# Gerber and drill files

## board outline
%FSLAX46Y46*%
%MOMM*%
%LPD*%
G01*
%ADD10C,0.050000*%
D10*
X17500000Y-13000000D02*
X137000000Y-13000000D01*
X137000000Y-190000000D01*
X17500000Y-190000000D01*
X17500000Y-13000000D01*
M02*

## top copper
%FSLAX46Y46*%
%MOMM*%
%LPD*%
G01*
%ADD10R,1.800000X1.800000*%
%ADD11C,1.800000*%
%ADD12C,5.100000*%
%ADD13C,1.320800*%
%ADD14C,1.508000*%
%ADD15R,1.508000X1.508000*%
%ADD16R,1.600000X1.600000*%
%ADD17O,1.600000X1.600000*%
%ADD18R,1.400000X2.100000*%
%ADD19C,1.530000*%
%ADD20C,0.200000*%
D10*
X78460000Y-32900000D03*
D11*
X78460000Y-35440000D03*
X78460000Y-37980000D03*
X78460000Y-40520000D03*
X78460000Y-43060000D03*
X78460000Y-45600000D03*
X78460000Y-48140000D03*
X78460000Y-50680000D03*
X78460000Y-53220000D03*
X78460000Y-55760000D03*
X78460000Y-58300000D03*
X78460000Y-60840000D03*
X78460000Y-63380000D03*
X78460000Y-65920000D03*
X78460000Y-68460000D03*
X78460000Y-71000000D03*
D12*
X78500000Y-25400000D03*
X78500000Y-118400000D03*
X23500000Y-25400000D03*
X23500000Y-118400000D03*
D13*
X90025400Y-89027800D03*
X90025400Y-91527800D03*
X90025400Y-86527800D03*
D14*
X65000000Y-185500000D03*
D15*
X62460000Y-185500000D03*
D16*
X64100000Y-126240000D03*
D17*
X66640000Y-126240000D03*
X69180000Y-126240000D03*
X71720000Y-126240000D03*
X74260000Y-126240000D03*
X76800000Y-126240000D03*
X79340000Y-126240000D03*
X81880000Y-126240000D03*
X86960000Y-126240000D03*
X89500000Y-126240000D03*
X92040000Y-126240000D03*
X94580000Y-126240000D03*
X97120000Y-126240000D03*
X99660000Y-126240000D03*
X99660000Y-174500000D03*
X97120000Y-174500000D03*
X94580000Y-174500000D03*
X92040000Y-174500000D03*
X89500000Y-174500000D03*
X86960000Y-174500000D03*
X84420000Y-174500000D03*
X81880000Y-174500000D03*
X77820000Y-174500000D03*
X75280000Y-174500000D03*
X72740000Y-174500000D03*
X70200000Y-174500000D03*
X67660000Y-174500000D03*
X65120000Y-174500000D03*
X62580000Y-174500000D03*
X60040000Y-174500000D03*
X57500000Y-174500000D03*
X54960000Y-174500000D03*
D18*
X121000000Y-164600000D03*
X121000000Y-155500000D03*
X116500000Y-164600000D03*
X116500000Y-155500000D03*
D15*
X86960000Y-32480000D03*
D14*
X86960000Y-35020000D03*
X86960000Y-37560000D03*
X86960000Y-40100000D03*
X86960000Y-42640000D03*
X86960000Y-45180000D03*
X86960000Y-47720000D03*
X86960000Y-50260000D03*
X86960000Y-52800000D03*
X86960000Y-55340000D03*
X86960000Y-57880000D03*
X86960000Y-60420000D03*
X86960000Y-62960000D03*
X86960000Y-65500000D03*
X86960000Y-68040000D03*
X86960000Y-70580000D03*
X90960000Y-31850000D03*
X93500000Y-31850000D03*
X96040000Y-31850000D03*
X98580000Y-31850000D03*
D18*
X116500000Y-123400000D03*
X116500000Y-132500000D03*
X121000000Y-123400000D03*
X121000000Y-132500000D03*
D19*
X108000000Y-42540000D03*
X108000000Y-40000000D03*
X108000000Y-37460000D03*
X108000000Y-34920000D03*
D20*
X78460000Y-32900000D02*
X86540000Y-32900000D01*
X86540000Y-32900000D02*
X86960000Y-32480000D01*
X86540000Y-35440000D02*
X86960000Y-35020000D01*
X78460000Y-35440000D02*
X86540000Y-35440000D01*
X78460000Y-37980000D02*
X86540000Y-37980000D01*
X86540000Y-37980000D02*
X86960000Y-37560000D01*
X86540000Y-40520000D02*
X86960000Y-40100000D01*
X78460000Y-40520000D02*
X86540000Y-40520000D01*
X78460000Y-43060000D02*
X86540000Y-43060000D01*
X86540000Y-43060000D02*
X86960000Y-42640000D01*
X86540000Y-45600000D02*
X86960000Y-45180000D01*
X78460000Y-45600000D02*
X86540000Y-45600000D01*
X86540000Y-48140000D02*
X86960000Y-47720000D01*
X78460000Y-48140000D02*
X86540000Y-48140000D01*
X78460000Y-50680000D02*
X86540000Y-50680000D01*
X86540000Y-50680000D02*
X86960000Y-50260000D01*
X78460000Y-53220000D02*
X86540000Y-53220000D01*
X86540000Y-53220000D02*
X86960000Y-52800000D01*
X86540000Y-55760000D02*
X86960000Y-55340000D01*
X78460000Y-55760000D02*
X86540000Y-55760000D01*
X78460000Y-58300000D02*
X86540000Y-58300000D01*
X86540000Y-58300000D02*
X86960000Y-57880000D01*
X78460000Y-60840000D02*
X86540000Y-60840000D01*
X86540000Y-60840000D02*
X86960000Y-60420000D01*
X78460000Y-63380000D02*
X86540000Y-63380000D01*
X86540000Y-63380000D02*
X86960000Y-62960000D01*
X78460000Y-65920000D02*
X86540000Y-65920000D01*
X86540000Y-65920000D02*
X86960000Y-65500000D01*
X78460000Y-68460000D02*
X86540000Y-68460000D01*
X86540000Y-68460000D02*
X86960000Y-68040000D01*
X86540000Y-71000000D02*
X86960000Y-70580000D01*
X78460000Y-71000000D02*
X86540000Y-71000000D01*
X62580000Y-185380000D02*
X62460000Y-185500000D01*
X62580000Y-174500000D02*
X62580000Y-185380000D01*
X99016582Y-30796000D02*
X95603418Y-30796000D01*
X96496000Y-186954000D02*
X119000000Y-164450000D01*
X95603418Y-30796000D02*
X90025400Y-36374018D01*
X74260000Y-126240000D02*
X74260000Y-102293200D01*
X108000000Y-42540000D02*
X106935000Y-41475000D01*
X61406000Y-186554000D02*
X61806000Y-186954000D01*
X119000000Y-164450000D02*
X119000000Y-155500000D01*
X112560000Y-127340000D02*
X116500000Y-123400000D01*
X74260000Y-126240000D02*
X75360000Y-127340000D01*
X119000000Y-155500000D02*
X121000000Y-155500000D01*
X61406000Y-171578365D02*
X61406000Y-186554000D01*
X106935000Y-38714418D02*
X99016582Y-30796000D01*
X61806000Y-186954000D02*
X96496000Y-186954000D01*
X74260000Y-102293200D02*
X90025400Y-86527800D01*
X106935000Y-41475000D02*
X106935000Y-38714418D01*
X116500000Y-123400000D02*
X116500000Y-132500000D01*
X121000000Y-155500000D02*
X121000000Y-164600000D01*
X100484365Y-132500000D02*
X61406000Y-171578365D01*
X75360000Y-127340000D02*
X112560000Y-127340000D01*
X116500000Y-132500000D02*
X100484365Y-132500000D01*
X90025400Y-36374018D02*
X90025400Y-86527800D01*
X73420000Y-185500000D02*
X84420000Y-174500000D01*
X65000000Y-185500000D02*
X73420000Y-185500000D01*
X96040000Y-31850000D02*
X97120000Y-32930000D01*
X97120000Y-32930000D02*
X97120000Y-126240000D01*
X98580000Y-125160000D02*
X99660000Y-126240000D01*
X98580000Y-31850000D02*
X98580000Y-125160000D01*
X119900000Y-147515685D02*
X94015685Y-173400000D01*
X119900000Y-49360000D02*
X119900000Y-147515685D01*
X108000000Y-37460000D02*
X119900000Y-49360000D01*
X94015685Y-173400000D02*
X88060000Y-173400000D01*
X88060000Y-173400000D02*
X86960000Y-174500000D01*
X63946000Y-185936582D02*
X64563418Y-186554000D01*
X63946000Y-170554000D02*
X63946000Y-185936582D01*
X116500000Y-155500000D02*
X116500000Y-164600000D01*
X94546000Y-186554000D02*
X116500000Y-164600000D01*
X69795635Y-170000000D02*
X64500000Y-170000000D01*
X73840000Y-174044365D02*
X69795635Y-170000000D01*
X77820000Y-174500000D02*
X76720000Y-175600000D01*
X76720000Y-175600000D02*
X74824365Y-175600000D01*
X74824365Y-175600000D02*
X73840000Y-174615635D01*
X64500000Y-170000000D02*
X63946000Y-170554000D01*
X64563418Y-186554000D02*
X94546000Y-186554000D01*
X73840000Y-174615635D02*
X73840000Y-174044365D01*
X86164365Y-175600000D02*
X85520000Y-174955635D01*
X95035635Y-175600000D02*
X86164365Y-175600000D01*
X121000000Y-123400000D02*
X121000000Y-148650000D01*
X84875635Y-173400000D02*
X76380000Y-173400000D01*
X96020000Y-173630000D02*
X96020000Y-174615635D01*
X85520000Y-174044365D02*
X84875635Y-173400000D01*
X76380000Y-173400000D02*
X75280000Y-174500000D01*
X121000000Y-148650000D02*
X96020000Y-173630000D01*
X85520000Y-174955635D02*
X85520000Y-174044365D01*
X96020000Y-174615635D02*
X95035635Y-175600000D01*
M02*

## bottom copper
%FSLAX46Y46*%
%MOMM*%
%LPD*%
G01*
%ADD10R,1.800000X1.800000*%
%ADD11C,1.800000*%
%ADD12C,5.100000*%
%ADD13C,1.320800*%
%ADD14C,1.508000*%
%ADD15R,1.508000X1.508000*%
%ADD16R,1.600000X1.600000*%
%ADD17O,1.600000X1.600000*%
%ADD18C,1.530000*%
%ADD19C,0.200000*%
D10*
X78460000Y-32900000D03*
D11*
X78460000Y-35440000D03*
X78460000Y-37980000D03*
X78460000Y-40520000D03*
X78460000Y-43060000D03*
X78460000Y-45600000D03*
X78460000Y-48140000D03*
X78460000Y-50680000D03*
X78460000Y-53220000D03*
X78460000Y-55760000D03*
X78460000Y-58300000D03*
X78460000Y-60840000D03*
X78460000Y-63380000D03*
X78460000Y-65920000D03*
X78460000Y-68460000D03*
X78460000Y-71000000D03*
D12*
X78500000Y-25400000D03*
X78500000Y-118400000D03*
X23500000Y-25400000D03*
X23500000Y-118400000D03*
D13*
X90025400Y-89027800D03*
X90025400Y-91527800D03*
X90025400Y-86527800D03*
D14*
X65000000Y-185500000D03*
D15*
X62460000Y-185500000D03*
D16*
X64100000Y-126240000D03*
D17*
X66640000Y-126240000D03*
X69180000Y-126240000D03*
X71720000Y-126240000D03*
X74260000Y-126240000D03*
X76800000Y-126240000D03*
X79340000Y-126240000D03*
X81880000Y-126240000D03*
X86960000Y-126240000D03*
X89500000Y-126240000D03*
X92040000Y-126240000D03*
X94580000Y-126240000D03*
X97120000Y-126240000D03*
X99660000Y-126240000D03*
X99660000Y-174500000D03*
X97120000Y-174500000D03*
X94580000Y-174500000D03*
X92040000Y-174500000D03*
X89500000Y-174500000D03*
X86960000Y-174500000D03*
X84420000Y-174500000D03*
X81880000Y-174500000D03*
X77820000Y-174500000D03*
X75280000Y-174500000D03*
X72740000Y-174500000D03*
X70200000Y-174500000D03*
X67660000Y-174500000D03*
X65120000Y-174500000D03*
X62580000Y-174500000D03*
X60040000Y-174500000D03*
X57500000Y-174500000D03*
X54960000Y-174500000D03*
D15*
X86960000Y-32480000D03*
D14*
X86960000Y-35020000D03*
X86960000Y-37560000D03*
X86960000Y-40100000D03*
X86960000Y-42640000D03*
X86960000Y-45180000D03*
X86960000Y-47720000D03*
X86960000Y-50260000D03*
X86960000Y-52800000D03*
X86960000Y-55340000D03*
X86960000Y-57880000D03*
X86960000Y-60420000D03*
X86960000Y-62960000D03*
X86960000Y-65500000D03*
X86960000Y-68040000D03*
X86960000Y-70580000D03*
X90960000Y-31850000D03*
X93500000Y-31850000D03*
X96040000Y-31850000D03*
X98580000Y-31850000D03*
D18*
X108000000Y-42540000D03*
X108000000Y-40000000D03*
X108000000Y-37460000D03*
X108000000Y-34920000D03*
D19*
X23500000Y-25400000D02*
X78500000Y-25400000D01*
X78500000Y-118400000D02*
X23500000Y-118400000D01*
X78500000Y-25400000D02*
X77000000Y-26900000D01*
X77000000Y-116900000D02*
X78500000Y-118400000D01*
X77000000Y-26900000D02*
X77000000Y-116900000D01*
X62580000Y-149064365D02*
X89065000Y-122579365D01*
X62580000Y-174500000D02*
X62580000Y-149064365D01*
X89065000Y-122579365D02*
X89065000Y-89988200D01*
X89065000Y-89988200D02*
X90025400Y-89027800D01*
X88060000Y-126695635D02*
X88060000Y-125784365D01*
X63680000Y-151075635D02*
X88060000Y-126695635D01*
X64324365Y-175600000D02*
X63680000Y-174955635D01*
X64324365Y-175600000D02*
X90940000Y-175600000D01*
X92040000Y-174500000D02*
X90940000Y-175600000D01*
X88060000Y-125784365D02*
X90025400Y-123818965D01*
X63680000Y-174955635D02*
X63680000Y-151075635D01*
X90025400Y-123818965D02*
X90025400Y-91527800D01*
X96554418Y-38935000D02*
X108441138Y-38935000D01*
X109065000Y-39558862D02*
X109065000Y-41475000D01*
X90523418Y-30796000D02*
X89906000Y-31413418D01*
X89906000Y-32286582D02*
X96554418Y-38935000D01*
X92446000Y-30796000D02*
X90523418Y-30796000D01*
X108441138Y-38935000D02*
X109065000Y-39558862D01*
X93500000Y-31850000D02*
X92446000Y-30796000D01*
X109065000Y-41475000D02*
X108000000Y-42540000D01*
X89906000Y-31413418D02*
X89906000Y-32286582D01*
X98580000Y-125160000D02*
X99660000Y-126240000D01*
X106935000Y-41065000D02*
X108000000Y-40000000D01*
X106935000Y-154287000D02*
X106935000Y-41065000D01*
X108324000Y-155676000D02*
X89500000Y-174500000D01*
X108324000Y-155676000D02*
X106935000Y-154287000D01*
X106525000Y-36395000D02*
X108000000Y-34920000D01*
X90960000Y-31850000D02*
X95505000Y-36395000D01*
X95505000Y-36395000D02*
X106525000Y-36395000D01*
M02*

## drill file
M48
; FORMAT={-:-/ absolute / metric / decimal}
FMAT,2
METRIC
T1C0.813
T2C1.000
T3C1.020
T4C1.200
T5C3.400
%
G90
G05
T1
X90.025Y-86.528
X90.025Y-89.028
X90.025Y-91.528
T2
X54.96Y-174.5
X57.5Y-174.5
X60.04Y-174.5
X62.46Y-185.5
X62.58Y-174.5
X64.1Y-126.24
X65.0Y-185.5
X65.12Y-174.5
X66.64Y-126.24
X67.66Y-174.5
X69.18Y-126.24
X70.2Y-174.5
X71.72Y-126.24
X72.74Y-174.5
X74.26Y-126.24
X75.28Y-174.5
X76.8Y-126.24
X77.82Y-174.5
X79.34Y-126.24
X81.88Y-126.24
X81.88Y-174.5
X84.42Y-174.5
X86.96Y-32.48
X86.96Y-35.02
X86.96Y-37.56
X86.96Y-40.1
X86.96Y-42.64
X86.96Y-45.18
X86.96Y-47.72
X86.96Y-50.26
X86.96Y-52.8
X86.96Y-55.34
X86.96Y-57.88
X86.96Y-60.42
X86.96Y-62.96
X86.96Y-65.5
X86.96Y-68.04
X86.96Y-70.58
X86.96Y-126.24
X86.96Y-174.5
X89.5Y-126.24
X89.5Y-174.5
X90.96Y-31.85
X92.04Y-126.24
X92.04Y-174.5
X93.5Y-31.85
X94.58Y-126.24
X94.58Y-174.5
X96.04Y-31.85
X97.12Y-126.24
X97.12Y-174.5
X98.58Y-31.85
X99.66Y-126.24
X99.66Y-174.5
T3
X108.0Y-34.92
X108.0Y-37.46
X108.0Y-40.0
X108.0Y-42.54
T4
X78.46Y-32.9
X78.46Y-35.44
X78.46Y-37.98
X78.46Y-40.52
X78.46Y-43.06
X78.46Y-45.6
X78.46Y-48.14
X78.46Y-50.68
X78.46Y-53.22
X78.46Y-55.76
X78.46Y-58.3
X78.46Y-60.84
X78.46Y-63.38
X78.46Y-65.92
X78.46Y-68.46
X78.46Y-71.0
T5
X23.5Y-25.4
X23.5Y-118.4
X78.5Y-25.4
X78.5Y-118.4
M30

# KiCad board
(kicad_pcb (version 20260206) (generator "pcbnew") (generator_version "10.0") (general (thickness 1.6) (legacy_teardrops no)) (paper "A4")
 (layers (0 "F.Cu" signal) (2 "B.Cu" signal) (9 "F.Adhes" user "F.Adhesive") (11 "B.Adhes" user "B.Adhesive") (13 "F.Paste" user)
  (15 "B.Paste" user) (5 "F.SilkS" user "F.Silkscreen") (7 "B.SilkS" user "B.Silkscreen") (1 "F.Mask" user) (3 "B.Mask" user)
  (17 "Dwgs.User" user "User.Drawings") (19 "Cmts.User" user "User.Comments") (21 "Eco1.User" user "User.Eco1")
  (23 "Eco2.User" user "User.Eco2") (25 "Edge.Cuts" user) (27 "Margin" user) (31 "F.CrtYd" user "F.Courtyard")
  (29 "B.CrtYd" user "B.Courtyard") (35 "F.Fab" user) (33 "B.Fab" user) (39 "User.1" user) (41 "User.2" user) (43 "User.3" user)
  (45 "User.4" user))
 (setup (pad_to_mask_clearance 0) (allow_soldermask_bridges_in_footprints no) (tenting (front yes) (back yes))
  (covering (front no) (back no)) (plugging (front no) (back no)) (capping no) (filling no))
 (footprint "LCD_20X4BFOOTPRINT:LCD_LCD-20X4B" (layer "F.Cu") (at 51 71.9 -90)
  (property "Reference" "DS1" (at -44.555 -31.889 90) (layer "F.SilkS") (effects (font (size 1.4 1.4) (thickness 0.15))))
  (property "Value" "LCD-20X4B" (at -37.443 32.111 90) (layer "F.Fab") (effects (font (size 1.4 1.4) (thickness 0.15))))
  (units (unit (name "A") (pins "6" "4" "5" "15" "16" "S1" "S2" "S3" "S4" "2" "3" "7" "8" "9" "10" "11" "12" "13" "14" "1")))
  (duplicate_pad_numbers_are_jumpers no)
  (pad "1" thru_hole rect (at -39 -27.46 270) (size 1.8 1.8) (drill 1.2) (layers "*.Cu" "*.Mask") (remove_unused_layers no)
   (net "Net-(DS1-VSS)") (solder_mask_margin 0.102))
  (pad "2" thru_hole circle (at -36.46 -27.46 270) (size 1.8 1.8) (drill 1.2) (layers "*.Cu" "*.Mask") (remove_unused_layers no)
   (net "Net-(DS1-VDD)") (solder_mask_margin 0.102))
  (pad "3" thru_hole circle (at -33.92 -27.46 270) (size 1.8 1.8) (drill 1.2) (layers "*.Cu" "*.Mask") (remove_unused_layers no)
   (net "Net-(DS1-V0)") (solder_mask_margin 0.102))
  (pad "4" thru_hole circle (at -31.38 -27.46 270) (size 1.8 1.8) (drill 1.2) (layers "*.Cu" "*.Mask") (remove_unused_layers no)
   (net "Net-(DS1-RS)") (solder_mask_margin 0.102))
  (pad "5" thru_hole circle (at -28.84 -27.46 270) (size 1.8 1.8) (drill 1.2) (layers "*.Cu" "*.Mask") (remove_unused_layers no)
   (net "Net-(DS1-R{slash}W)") (solder_mask_margin 0.102))
  (pad "6" thru_hole circle (at -26.3 -27.46 270) (size 1.8 1.8) (drill 1.2) (layers "*.Cu" "*.Mask") (remove_unused_layers no)
   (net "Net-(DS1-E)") (solder_mask_margin 0.102))
  (pad "7" thru_hole circle (at -23.76 -27.46 270) (size 1.8 1.8) (drill 1.2) (layers "*.Cu" "*.Mask") (remove_unused_layers no)
   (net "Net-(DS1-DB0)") (solder_mask_margin 0.102))
  (pad "8" thru_hole circle (at -21.22 -27.46 270) (size 1.8 1.8) (drill 1.2) (layers "*.Cu" "*.Mask") (remove_unused_layers no)
   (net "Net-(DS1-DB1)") (solder_mask_margin 0.102))
  (pad "9" thru_hole circle (at -18.68 -27.46 270) (size 1.8 1.8) (drill 1.2) (layers "*.Cu" "*.Mask") (remove_unused_layers no)
   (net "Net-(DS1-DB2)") (solder_mask_margin 0.102))
  (pad "10" thru_hole circle (at -16.14 -27.46 270) (size 1.8 1.8) (drill 1.2) (layers "*.Cu" "*.Mask") (remove_unused_layers no)
   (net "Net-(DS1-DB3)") (solder_mask_margin 0.102))
  (pad "11" thru_hole circle (at -13.6 -27.46 270) (size 1.8 1.8) (drill 1.2) (layers "*.Cu" "*.Mask") (remove_unused_layers no)
   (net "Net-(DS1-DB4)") (solder_mask_margin 0.102))
  (pad "12" thru_hole circle (at -11.06 -27.46 270) (size 1.8 1.8) (drill 1.2) (layers "*.Cu" "*.Mask") (remove_unused_layers no)
   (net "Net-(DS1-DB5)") (solder_mask_margin 0.102))
  (pad "13" thru_hole circle (at -8.52 -27.46 270) (size 1.8 1.8) (drill 1.2) (layers "*.Cu" "*.Mask") (remove_unused_layers no)
   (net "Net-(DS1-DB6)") (solder_mask_margin 0.102))
  (pad "14" thru_hole circle (at -5.98 -27.46 270) (size 1.8 1.8) (drill 1.2) (layers "*.Cu" "*.Mask") (remove_unused_layers no)
   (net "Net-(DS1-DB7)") (solder_mask_margin 0.102))
  (pad "15" thru_hole circle (at -3.44 -27.46 270) (size 1.8 1.8) (drill 1.2) (layers "*.Cu" "*.Mask") (remove_unused_layers no)
   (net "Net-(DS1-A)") (solder_mask_margin 0.102))
  (pad "16" thru_hole circle (at -0.9 -27.46 270) (size 1.8 1.8) (drill 1.2) (layers "*.Cu" "*.Mask") (remove_unused_layers no)
   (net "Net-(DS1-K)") (solder_mask_margin 0.102))
  (pad "S1" thru_hole circle (at -46.5 -27.5 270) (size 5.1 5.1) (drill 3.4) (layers "*.Cu" "*.Mask") (remove_unused_layers no)
   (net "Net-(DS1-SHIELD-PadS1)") (solder_mask_margin 0.102))
  (pad "S2" thru_hole circle (at 46.5 -27.5 270) (size 5.1 5.1) (drill 3.4) (layers "*.Cu" "*.Mask") (remove_unused_layers no)
   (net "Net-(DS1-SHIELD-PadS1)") (solder_mask_margin 0.102))
  (pad "S3" thru_hole circle (at -46.5 27.5 270) (size 5.1 5.1) (drill 3.4) (layers "*.Cu" "*.Mask") (remove_unused_layers no)
   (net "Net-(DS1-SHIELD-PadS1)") (solder_mask_margin 0.102))
  (pad "S4" thru_hole circle (at 46.5 27.5 270) (size 5.1 5.1) (drill 3.4) (layers "*.Cu" "*.Mask") (remove_unused_layers no)
   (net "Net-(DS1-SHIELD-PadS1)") (solder_mask_margin 0.102)))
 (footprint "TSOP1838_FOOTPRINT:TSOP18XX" (layer "F.Cu") (at 89.9988 89.0266 90)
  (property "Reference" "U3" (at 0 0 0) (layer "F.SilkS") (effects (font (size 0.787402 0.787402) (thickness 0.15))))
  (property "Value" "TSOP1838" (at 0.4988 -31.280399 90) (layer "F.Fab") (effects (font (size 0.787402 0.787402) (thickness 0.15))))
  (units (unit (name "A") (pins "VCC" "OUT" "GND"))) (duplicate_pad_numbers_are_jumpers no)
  (pad "GND" thru_hole circle (at -0.0012 0.0266 90) (size 1.3208 1.3208) (drill 0.8128) (layers "*.Cu" "*.Mask") (remove_unused_layers no)
   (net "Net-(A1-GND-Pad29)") (solder_mask_margin 0.102))
  (pad "OUT" thru_hole circle (at -2.5012 0.0266 90) (size 1.3208 1.3208) (drill 0.8128) (layers "*.Cu" "*.Mask") (remove_unused_layers no)
   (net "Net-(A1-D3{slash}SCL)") (solder_mask_margin 0.102))
  (pad "VCC" thru_hole circle (at 2.4988 0.0266 90) (size 1.3208 1.3208) (drill 0.8128) (layers "*.Cu" "*.Mask") (remove_unused_layers no)
   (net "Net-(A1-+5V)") (solder_mask_margin 0.102)))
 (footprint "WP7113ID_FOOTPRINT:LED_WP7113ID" (layer "F.Cu") (at 63.73 185.5)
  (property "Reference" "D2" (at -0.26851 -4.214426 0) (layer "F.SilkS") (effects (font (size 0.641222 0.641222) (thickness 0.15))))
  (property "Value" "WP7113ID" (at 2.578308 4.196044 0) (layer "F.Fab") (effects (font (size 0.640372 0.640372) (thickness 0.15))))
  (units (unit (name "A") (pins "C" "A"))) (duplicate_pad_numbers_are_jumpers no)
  (pad "A" thru_hole circle (at 1.27 0) (size 1.508 1.508) (drill 1) (layers "*.Cu" "*.Mask") (remove_unused_layers no) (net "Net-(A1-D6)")
   (solder_mask_margin 0.102))
  (pad "C" thru_hole rect (at -1.27 0) (size 1.508 1.508) (drill 1) (layers "*.Cu" "*.Mask") (remove_unused_layers no)
   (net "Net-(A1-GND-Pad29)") (solder_mask_margin 0.102)))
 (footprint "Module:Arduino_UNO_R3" (layer "F.Cu") (at 64.1 126.24)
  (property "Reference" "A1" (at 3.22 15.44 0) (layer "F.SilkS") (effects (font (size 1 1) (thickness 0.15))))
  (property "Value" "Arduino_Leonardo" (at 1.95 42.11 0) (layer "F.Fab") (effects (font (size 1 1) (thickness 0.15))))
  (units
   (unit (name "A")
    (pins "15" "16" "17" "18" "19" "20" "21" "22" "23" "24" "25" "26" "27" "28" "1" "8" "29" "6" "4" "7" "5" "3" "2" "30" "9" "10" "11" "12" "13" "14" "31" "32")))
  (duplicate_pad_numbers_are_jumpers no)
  (pad "1" thru_hole rect (at 0 0 90) (size 1.6 1.6) (drill 1) (layers "*.Cu" "*.Mask") (remove_unused_layers no)
   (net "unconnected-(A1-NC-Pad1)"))
  (pad "2" thru_hole oval (at 2.54 0 90) (size 1.6 1.6) (drill 1) (layers "*.Cu" "*.Mask") (remove_unused_layers no)
   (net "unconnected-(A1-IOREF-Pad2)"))
  (pad "3" thru_hole oval (at 5.08 0 90) (size 1.6 1.6) (drill 1) (layers "*.Cu" "*.Mask") (remove_unused_layers no)
   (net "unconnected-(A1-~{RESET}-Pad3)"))
  (pad "4" thru_hole oval (at 7.62 0 90) (size 1.6 1.6) (drill 1) (layers "*.Cu" "*.Mask") (remove_unused_layers no)
   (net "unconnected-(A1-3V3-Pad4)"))
  (pad "5" thru_hole oval (at 10.16 0 90) (size 1.6 1.6) (drill 1) (layers "*.Cu" "*.Mask") (remove_unused_layers no) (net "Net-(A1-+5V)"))
  (pad "6" thru_hole oval (at 12.7 0 90) (size 1.6 1.6) (drill 1) (layers "*.Cu" "*.Mask") (remove_unused_layers no)
   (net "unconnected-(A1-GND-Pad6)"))
  (pad "7" thru_hole oval (at 15.24 0 90) (size 1.6 1.6) (drill 1) (layers "*.Cu" "*.Mask") (remove_unused_layers no)
   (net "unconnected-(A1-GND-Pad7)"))
  (pad "8" thru_hole oval (at 17.78 0 90) (size 1.6 1.6) (drill 1) (layers "*.Cu" "*.Mask") (remove_unused_layers no)
   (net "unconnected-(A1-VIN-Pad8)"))
  (pad "9" thru_hole oval (at 22.86 0 90) (size 1.6 1.6) (drill 1) (layers "*.Cu" "*.Mask") (remove_unused_layers no)
   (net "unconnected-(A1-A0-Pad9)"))
  (pad "10" thru_hole oval (at 25.4 0 90) (size 1.6 1.6) (drill 1) (layers "*.Cu" "*.Mask") (remove_unused_layers no)
   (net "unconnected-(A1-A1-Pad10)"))
  (pad "11" thru_hole oval (at 27.94 0 90) (size 1.6 1.6) (drill 1) (layers "*.Cu" "*.Mask") (remove_unused_layers no)
   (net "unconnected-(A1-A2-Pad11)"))
  (pad "12" thru_hole oval (at 30.48 0 90) (size 1.6 1.6) (drill 1) (layers "*.Cu" "*.Mask") (remove_unused_layers no)
   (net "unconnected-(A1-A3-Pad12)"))
  (pad "13" thru_hole oval (at 33.02 0 90) (size 1.6 1.6) (drill 1) (layers "*.Cu" "*.Mask") (remove_unused_layers no) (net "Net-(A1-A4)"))
  (pad "14" thru_hole oval (at 35.56 0 90) (size 1.6 1.6) (drill 1) (layers "*.Cu" "*.Mask") (remove_unused_layers no) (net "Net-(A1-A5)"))
  (pad "15" thru_hole oval (at 35.56 48.26 90) (size 1.6 1.6) (drill 1) (layers "*.Cu" "*.Mask") (remove_unused_layers no)
   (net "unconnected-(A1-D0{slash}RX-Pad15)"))
  (pad "16" thru_hole oval (at 33.02 48.26 90) (size 1.6 1.6) (drill 1) (layers "*.Cu" "*.Mask") (remove_unused_layers no)
   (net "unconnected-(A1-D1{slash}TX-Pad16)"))
  (pad "17" thru_hole oval (at 30.48 48.26 90) (size 1.6 1.6) (drill 1) (layers "*.Cu" "*.Mask") (remove_unused_layers no)
   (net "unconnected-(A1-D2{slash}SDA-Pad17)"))
  (pad "18" thru_hole oval (at 27.94 48.26 90) (size 1.6 1.6) (drill 1) (layers "*.Cu" "*.Mask") (remove_unused_layers no)
   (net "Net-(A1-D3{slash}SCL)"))
  (pad "19" thru_hole oval (at 25.4 48.26 90) (size 1.6 1.6) (drill 1) (layers "*.Cu" "*.Mask") (remove_unused_layers no)
   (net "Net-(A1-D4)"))
  (pad "20" thru_hole oval (at 22.86 48.26 90) (size 1.6 1.6) (drill 1) (layers "*.Cu" "*.Mask") (remove_unused_layers no)
   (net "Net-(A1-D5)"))
  (pad "21" thru_hole oval (at 20.32 48.26 90) (size 1.6 1.6) (drill 1) (layers "*.Cu" "*.Mask") (remove_unused_layers no)
   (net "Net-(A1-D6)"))
  (pad "22" thru_hole oval (at 17.78 48.26 90) (size 1.6 1.6) (drill 1) (layers "*.Cu" "*.Mask") (remove_unused_layers no)
   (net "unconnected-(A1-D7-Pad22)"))
  (pad "23" thru_hole oval (at 13.72 48.26 90) (size 1.6 1.6) (drill 1) (layers "*.Cu" "*.Mask") (remove_unused_layers no)
   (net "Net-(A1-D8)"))
  (pad "24" thru_hole oval (at 11.18 48.26 90) (size 1.6 1.6) (drill 1) (layers "*.Cu" "*.Mask") (remove_unused_layers no)
   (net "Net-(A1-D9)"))
  (pad "25" thru_hole oval (at 8.64 48.26 90) (size 1.6 1.6) (drill 1) (layers "*.Cu" "*.Mask") (remove_unused_layers no)
   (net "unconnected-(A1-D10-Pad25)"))
  (pad "26" thru_hole oval (at 6.1 48.26 90) (size 1.6 1.6) (drill 1) (layers "*.Cu" "*.Mask") (remove_unused_layers no)
   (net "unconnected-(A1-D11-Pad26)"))
  (pad "27" thru_hole oval (at 3.56 48.26 90) (size 1.6 1.6) (drill 1) (layers "*.Cu" "*.Mask") (remove_unused_layers no)
   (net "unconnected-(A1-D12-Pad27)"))
  (pad "28" thru_hole oval (at 1.02 48.26 90) (size 1.6 1.6) (drill 1) (layers "*.Cu" "*.Mask") (remove_unused_layers no)
   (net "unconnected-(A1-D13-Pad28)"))
  (pad "29" thru_hole oval (at -1.52 48.26 90) (size 1.6 1.6) (drill 1) (layers "*.Cu" "*.Mask") (remove_unused_layers no)
   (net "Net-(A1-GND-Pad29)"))
  (pad "30" thru_hole oval (at -4.06 48.26 90) (size 1.6 1.6) (drill 1) (layers "*.Cu" "*.Mask") (remove_unused_layers no)
   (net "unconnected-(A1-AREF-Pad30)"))
  (pad "31" thru_hole oval (at -6.6 48.26 90) (size 1.6 1.6) (drill 1) (layers "*.Cu" "*.Mask") (remove_unused_layers no)
   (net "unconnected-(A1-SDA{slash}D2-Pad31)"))
  (pad "32" thru_hole oval (at -9.14 48.26 90) (size 1.6 1.6) (drill 1) (layers "*.Cu" "*.Mask") (remove_unused_layers no)
   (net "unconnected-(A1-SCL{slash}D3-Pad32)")))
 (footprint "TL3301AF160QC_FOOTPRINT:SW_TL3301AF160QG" (layer "F.Cu") (at 118.75 160.05 90)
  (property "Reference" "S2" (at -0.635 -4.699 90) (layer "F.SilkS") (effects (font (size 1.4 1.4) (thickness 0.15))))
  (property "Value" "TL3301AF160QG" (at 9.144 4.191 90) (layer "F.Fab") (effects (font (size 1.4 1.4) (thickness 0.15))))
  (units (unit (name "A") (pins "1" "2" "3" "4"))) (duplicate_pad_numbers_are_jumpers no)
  (pad "1" smd rect (at -4.55 2.25 90) (size 2.1 1.4) (layers "F.Cu" "F.Mask" "F.Paste") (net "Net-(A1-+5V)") (solder_mask_margin 0.102))
  (pad "2" smd rect (at 4.55 2.25 90) (size 2.1 1.4) (layers "F.Cu" "F.Mask" "F.Paste") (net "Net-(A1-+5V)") (solder_mask_margin 0.102))
  (pad "3" smd rect (at -4.55 -2.25 90) (size 2.1 1.4) (layers "F.Cu" "F.Mask" "F.Paste") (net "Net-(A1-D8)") (solder_mask_margin 0.102))
  (pad "4" smd rect (at 4.55 -2.25 90) (size 2.1 1.4) (layers "F.Cu" "F.Mask" "F.Paste") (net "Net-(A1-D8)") (solder_mask_margin 0.102)))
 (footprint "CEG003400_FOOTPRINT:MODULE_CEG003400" (layer "F.Cu") (at 94.71 51.315)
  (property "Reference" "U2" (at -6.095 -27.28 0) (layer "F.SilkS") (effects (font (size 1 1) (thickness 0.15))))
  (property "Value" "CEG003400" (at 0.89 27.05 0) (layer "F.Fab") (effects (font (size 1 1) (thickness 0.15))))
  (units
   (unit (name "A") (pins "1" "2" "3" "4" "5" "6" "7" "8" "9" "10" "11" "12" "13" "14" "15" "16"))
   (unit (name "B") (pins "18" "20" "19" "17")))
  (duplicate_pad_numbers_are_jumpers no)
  (pad "1" thru_hole rect (at -7.75 -18.835) (size 1.508 1.508) (drill 1) (layers "*.Cu" "*.Mask") (remove_unused_layers no)
   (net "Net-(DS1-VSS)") (solder_mask_margin 0.102))
  (pad "2" thru_hole circle (at -7.75 -16.295) (size 1.508 1.508) (drill 1) (layers "*.Cu" "*.Mask") (remove_unused_layers no)
   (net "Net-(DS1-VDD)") (solder_mask_margin 0.102))
  (pad "3" thru_hole circle (at -7.75 -13.755) (size 1.508 1.508) (drill 1) (layers "*.Cu" "*.Mask") (remove_unused_layers no)
   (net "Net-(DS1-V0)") (solder_mask_margin 0.102))
  (pad "4" thru_hole circle (at -7.75 -11.215) (size 1.508 1.508) (drill 1) (layers "*.Cu" "*.Mask") (remove_unused_layers no)
   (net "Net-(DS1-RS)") (solder_mask_margin 0.102))
  (pad "5" thru_hole circle (at -7.75 -8.675) (size 1.508 1.508) (drill 1) (layers "*.Cu" "*.Mask") (remove_unused_layers no)
   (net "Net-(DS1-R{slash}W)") (solder_mask_margin 0.102))
  (pad "6" thru_hole circle (at -7.75 -6.135) (size 1.508 1.508) (drill 1) (layers "*.Cu" "*.Mask") (remove_unused_layers no)
   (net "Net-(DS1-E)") (solder_mask_margin 0.102))
  (pad "7" thru_hole circle (at -7.75 -3.595) (size 1.508 1.508) (drill 1) (layers "*.Cu" "*.Mask") (remove_unused_layers no)
   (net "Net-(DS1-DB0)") (solder_mask_margin 0.102))
  (pad "8" thru_hole circle (at -7.75 -1.055) (size 1.508 1.508) (drill 1) (layers "*.Cu" "*.Mask") (remove_unused_layers no)
   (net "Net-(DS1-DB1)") (solder_mask_margin 0.102))
  (pad "9" thru_hole circle (at -7.75 1.485) (size 1.508 1.508) (drill 1) (layers "*.Cu" "*.Mask") (remove_unused_layers no)
   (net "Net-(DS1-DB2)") (solder_mask_margin 0.102))
  (pad "10" thru_hole circle (at -7.75 4.025) (size 1.508 1.508) (drill 1) (layers "*.Cu" "*.Mask") (remove_unused_layers no)
   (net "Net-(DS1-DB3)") (solder_mask_margin 0.102))
  (pad "11" thru_hole circle (at -7.75 6.565) (size 1.508 1.508) (drill 1) (layers "*.Cu" "*.Mask") (remove_unused_layers no)
   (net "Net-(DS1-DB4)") (solder_mask_margin 0.102))
  (pad "12" thru_hole circle (at -7.75 9.105) (size 1.508 1.508) (drill 1) (layers "*.Cu" "*.Mask") (remove_unused_layers no)
   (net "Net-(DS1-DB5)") (solder_mask_margin 0.102))
  (pad "13" thru_hole circle (at -7.75 11.645) (size 1.508 1.508) (drill 1) (layers "*.Cu" "*.Mask") (remove_unused_layers no)
   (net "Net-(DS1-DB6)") (solder_mask_margin 0.102))
  (pad "14" thru_hole circle (at -7.75 14.185) (size 1.508 1.508) (drill 1) (layers "*.Cu" "*.Mask") (remove_unused_layers no)
   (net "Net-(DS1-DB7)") (solder_mask_margin 0.102))
  (pad "15" thru_hole circle (at -7.75 16.725) (size 1.508 1.508) (drill 1) (layers "*.Cu" "*.Mask") (remove_unused_layers no)
   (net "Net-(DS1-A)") (solder_mask_margin 0.102))
  (pad "16" thru_hole circle (at -7.75 19.265) (size 1.508 1.508) (drill 1) (layers "*.Cu" "*.Mask") (remove_unused_layers no)
   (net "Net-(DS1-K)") (solder_mask_margin 0.102))
  (pad "17" thru_hole circle (at -3.75 -19.465) (size 1.508 1.508) (drill 1) (layers "*.Cu" "*.Mask") (remove_unused_layers no)
   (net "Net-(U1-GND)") (solder_mask_margin 0.102))
  (pad "18" thru_hole circle (at -1.21 -19.465) (size 1.508 1.508) (drill 1) (layers "*.Cu" "*.Mask") (remove_unused_layers no)
   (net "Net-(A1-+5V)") (solder_mask_margin 0.102))
  (pad "19" thru_hole circle (at 1.33 -19.465) (size 1.508 1.508) (drill 1) (layers "*.Cu" "*.Mask") (remove_unused_layers no)
   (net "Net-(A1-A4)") (solder_mask_margin 0.102))
  (pad "20" thru_hole circle (at 3.87 -19.465) (size 1.508 1.508) (drill 1) (layers "*.Cu" "*.Mask") (remove_unused_layers no)
   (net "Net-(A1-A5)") (solder_mask_margin 0.102)))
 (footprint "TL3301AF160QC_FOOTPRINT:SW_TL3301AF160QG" (layer "F.Cu") (at 118.75 127.95 -90)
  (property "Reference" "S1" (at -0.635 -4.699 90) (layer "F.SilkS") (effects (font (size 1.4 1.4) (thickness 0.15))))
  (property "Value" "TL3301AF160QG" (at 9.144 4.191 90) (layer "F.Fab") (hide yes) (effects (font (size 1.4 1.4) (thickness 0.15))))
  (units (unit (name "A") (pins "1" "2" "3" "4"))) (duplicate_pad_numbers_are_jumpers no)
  (pad "1" smd rect (at -4.55 2.25 270) (size 2.1 1.4) (layers "F.Cu" "F.Mask" "F.Paste") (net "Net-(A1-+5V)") (solder_mask_margin 0.102))
  (pad "2" smd rect (at 4.55 2.25 270) (size 2.1 1.4) (layers "F.Cu" "F.Mask" "F.Paste") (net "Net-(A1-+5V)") (solder_mask_margin 0.102))
  (pad "3" smd rect (at -4.55 -2.25 270) (size 2.1 1.4) (layers "F.Cu" "F.Mask" "F.Paste") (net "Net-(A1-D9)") (solder_mask_margin 0.102))
  (pad "4" smd rect (at 4.55 -2.25 270) (size 2.1 1.4) (layers "F.Cu" "F.Mask" "F.Paste") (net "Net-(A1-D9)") (solder_mask_margin 0.102)))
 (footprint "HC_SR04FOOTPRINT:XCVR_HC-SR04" (layer "F.Cu") (at 108 38.73 90)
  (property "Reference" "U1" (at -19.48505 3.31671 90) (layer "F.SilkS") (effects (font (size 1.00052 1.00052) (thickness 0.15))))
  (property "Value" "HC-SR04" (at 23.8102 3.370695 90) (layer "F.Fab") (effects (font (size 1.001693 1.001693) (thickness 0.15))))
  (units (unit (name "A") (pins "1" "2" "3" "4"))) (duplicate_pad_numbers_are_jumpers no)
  (pad "1" thru_hole circle (at -3.81 0 90) (size 1.53 1.53) (drill 1.02) (layers "*.Cu" "*.Mask") (remove_unused_layers no)
   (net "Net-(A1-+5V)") (solder_mask_margin 0.102))
  (pad "2" thru_hole circle (at -1.27 0 90) (size 1.53 1.53) (drill 1.02) (layers "*.Cu" "*.Mask") (remove_unused_layers no)
   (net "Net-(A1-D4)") (solder_mask_margin 0.102))
  (pad "3" thru_hole circle (at 1.27 0 90) (size 1.53 1.53) (drill 1.02) (layers "*.Cu" "*.Mask") (remove_unused_layers no)
   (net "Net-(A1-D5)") (solder_mask_margin 0.102))
  (pad "4" thru_hole circle (at 3.81 0 90) (size 1.53 1.53) (drill 1.02) (layers "*.Cu" "*.Mask") (remove_unused_layers no)
   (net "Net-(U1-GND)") (solder_mask_margin 0.102)))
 (gr_poly (pts (xy 17.5 13) (xy 137 13) (xy 137 190) (xy 17.5 190)) (stroke (width 0.05) (type solid)) (fill no) (layer "Edge.Cuts"))
 (segment (start 78.46 32.9) (end 86.54 32.9) (width 0.2) (layer "F.Cu") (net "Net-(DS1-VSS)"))
 (segment (start 86.54 32.9) (end 86.96 32.48) (width 0.2) (layer "F.Cu") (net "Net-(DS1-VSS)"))
 (segment (start 86.54 35.44) (end 86.96 35.02) (width 0.2) (layer "F.Cu") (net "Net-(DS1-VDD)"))
 (segment (start 78.46 35.44) (end 86.54 35.44) (width 0.2) (layer "F.Cu") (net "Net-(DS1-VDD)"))
 (segment (start 78.46 37.98) (end 86.54 37.98) (width 0.2) (layer "F.Cu") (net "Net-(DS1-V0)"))
 (segment (start 86.54 37.98) (end 86.96 37.56) (width 0.2) (layer "F.Cu") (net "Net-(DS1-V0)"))
 (segment (start 86.54 40.52) (end 86.96 40.1) (width 0.2) (layer "F.Cu") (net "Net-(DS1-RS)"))
 (segment (start 78.46 40.52) (end 86.54 40.52) (width 0.2) (layer "F.Cu") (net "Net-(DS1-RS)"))
 (segment (start 78.46 43.06) (end 86.54 43.06) (width 0.2) (layer "F.Cu") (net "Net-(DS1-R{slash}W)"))
 (segment (start 86.54 43.06) (end 86.96 42.64) (width 0.2) (layer "F.Cu") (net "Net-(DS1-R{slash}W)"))
 (segment (start 86.54 45.6) (end 86.96 45.18) (width 0.2) (layer "F.Cu") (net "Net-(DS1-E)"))
 (segment (start 78.46 45.6) (end 86.54 45.6) (width 0.2) (layer "F.Cu") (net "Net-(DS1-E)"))
 (segment (start 86.54 48.14) (end 86.96 47.72) (width 0.2) (layer "F.Cu") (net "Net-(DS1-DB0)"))
 (segment (start 78.46 48.14) (end 86.54 48.14) (width 0.2) (layer "F.Cu") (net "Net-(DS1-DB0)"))
 (segment (start 78.46 50.68) (end 86.54 50.68) (width 0.2) (layer "F.Cu") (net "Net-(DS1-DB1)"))
 (segment (start 86.54 50.68) (end 86.96 50.26) (width 0.2) (layer "F.Cu") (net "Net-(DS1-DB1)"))
 (segment (start 78.46 53.22) (end 86.54 53.22) (width 0.2) (layer "F.Cu") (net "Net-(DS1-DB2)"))
 (segment (start 86.54 53.22) (end 86.96 52.8) (width 0.2) (layer "F.Cu") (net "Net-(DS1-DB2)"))
 (segment (start 86.54 55.76) (end 86.96 55.34) (width 0.2) (layer "F.Cu") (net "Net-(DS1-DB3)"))
 (segment (start 78.46 55.76) (end 86.54 55.76) (width 0.2) (layer "F.Cu") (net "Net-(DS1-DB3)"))
 (segment (start 78.46 58.3) (end 86.54 58.3) (width 0.2) (layer "F.Cu") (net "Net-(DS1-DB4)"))
 (segment (start 86.54 58.3) (end 86.96 57.88) (width 0.2) (layer "F.Cu") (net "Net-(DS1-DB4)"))
 (segment (start 78.46 60.84) (end 86.54 60.84) (width 0.2) (layer "F.Cu") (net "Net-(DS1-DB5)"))
 (segment (start 86.54 60.84) (end 86.96 60.42) (width 0.2) (layer "F.Cu") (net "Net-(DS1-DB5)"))
 (segment (start 78.46 63.38) (end 86.54 63.38) (width 0.2) (layer "F.Cu") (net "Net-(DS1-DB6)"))
 (segment (start 86.54 63.38) (end 86.96 62.96) (width 0.2) (layer "F.Cu") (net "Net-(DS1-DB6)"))
 (segment (start 78.46 65.92) (end 86.54 65.92) (width 0.2) (layer "F.Cu") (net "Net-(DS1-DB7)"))
 (segment (start 86.54 65.92) (end 86.96 65.5) (width 0.2) (layer "F.Cu") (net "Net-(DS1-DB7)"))
 (segment (start 78.46 68.46) (end 86.54 68.46) (width 0.2) (layer "F.Cu") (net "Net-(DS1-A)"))
 (segment (start 86.54 68.46) (end 86.96 68.04) (width 0.2) (layer "F.Cu") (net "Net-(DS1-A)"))
 (segment (start 86.54 71) (end 86.96 70.58) (width 0.2) (layer "F.Cu") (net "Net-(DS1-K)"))
 (segment (start 78.46 71) (end 86.54 71) (width 0.2) (layer "F.Cu") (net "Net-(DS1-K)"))
 (segment (start 23.5 25.4) (end 78.5 25.4) (width 0.2) (layer "B.Cu") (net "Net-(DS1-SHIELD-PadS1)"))
 (segment (start 78.5 118.4) (end 23.5 118.4) (width 0.2) (layer "B.Cu") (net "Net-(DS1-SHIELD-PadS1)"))
 (segment (start 78.5 25.4) (end 77 26.9) (width 0.2) (layer "B.Cu") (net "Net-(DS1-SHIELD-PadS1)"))
 (segment (start 77 116.9) (end 78.5 118.4) (width 0.2) (layer "B.Cu") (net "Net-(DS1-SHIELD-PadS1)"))
 (segment (start 77 26.9) (end 77 116.9) (width 0.2) (layer "B.Cu") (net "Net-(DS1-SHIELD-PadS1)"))
 (segment (start 62.58 185.38) (end 62.46 185.5) (width 0.2) (layer "F.Cu") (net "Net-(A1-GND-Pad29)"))
 (segment (start 62.58 174.5) (end 62.58 185.38) (width 0.2) (layer "F.Cu") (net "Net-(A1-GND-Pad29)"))
 (segment (start 62.58 149.064365) (end 89.065 122.579365) (width 0.2) (layer "B.Cu") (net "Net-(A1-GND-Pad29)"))
 (segment (start 62.58 174.5) (end 62.58 149.064365) (width 0.2) (layer "B.Cu") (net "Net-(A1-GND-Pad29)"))
 (segment (start 89.065 122.579365) (end 89.065 89.9882) (width 0.2) (layer "B.Cu") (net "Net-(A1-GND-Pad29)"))
 (segment (start 89.065 89.9882) (end 90.0254 89.0278) (width 0.2) (layer "B.Cu") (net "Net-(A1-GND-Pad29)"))
 (segment (start 88.06 126.695635) (end 88.06 125.784365) (width 0.2) (layer "B.Cu") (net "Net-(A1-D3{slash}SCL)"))
 (segment (start 63.68 151.075635) (end 88.06 126.695635) (width 0.2) (layer "B.Cu") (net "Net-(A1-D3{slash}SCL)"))
 (segment (start 64.324365 175.6) (end 63.68 174.955635) (width 0.2) (layer "B.Cu") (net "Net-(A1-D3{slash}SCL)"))
 (segment (start 64.324365 175.6) (end 90.94 175.6) (width 0.2) (layer "B.Cu") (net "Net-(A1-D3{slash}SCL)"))
 (segment (start 92.04 174.5) (end 90.94 175.6) (width 0.2) (layer "B.Cu") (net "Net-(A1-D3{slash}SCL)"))
 (segment (start 88.06 125.784365) (end 90.0254 123.818965) (width 0.2) (layer "B.Cu") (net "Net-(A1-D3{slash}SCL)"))
 (segment (start 63.68 174.955635) (end 63.68 151.075635) (width 0.2) (layer "B.Cu") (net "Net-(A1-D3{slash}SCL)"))
 (segment (start 90.0254 123.818965) (end 90.0254 91.5278) (width 0.2) (layer "B.Cu") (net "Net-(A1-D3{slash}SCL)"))
 (segment (start 99.016582 30.796) (end 95.603418 30.796) (width 0.2) (layer "F.Cu") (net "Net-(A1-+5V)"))
 (segment (start 96.496 186.954) (end 119 164.45) (width 0.2) (layer "F.Cu") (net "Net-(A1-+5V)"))
 (segment (start 95.603418 30.796) (end 90.0254 36.374018) (width 0.2) (layer "F.Cu") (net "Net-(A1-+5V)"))
 (segment (start 74.26 126.24) (end 74.26 102.2932) (width 0.2) (layer "F.Cu") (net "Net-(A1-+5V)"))
 (segment (start 108 42.54) (end 106.935 41.475) (width 0.2) (layer "F.Cu") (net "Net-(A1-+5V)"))
 (segment (start 61.406 186.554) (end 61.806 186.954) (width 0.2) (layer "F.Cu") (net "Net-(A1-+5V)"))
 (segment (start 119 164.45) (end 119 155.5) (width 0.2) (layer "F.Cu") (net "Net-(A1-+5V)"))
 (segment (start 112.56 127.34) (end 116.5 123.4) (width 0.2) (layer "F.Cu") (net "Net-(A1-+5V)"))
 (segment (start 74.26 126.24) (end 75.36 127.34) (width 0.2) (layer "F.Cu") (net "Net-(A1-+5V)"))
 (segment (start 119 155.5) (end 121 155.5) (width 0.2) (layer "F.Cu") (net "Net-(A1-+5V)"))
 (segment (start 61.406 171.578365) (end 61.406 186.554) (width 0.2) (layer "F.Cu") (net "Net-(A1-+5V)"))
 (segment (start 106.935 38.714418) (end 99.016582 30.796) (width 0.2) (layer "F.Cu") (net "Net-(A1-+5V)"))
 (segment (start 61.806 186.954) (end 96.496 186.954) (width 0.2) (layer "F.Cu") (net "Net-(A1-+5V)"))
 (segment (start 74.26 102.2932) (end 90.0254 86.5278) (width 0.2) (layer "F.Cu") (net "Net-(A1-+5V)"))
 (segment (start 106.935 41.475) (end 106.935 38.714418) (width 0.2) (layer "F.Cu") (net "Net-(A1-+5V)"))
 (segment (start 116.5 123.4) (end 116.5 132.5) (width 0.2) (layer "F.Cu") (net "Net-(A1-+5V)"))
 (segment (start 121 155.5) (end 121 164.6) (width 0.2) (layer "F.Cu") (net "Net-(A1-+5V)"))
 (segment (start 100.484365 132.5) (end 61.406 171.578365) (width 0.2) (layer "F.Cu") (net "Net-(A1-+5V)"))
 (segment (start 75.36 127.34) (end 112.56 127.34) (width 0.2) (layer "F.Cu") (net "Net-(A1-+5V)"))
 (segment (start 116.5 132.5) (end 100.484365 132.5) (width 0.2) (layer "F.Cu") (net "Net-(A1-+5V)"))
 (segment (start 90.0254 36.374018) (end 90.0254 86.5278) (width 0.2) (layer "F.Cu") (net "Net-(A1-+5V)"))
 (segment (start 96.554418 38.935) (end 108.441138 38.935) (width 0.2) (layer "B.Cu") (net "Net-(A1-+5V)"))
 (segment (start 109.065 39.558862) (end 109.065 41.475) (width 0.2) (layer "B.Cu") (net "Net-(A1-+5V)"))
 (segment (start 90.523418 30.796) (end 89.906 31.413418) (width 0.2) (layer "B.Cu") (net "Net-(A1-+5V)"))
 (segment (start 89.906 32.286582) (end 96.554418 38.935) (width 0.2) (layer "B.Cu") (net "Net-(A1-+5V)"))
 (segment (start 92.446 30.796) (end 90.523418 30.796) (width 0.2) (layer "B.Cu") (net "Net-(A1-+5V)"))
 (segment (start 108.441138 38.935) (end 109.065 39.558862) (width 0.2) (layer "B.Cu") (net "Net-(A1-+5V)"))
 (segment (start 93.5 31.85) (end 92.446 30.796) (width 0.2) (layer "B.Cu") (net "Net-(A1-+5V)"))
 (segment (start 109.065 41.475) (end 108 42.54) (width 0.2) (layer "B.Cu") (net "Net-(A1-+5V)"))
 (segment (start 89.906 31.413418) (end 89.906 32.286582) (width 0.2) (layer "B.Cu") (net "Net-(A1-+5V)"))
 (segment (start 73.42 185.5) (end 84.42 174.5) (width 0.2) (layer "F.Cu") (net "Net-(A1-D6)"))
 (segment (start 65 185.5) (end 73.42 185.5) (width 0.2) (layer "F.Cu") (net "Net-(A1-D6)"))
 (segment (start 96.04 31.85) (end 97.12 32.93) (width 0.2) (layer "F.Cu") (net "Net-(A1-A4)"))
 (segment (start 97.12 32.93) (end 97.12 126.24) (width 0.2) (layer "F.Cu") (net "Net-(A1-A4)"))
 (segment (start 98.58 125.16) (end 99.66 126.24) (width 0.2) (layer "F.Cu") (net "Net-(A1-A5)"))
 (segment (start 98.58 31.85) (end 98.58 125.16) (width 0.2) (layer "F.Cu") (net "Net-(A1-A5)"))
 (segment (start 98.58 125.16) (end 99.66 126.24) (width 0.2) (layer "B.Cu") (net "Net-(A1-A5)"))
 (segment (start 106.935 41.065) (end 108 40) (width 0.2) (layer "B.Cu") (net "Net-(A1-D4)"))
 (segment (start 106.935 154.287) (end 106.935 41.065) (width 0.2) (layer "B.Cu") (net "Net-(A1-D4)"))
 (segment (start 108.324 155.676) (end 89.5 174.5) (width 0.2) (layer "B.Cu") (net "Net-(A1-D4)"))
 (segment (start 108.324 155.676) (end 106.935 154.287) (width 0.2) (layer "B.Cu") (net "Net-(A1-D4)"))
 (segment (start 119.9 147.515685) (end 94.015685 173.4) (width 0.2) (layer "F.Cu") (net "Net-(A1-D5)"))
 (segment (start 119.9 49.36) (end 119.9 147.515685) (width 0.2) (layer "F.Cu") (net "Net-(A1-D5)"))
 (segment (start 108 37.46) (end 119.9 49.36) (width 0.2) (layer "F.Cu") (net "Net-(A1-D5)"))
 (segment (start 94.015685 173.4) (end 88.06 173.4) (width 0.2) (layer "F.Cu") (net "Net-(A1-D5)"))
 (segment (start 88.06 173.4) (end 86.96 174.5) (width 0.2) (layer "F.Cu") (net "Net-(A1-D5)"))
 (segment (start 63.946 185.936582) (end 64.563418 186.554) (width 0.2) (layer "F.Cu") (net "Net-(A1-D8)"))
 (segment (start 63.946 170.554) (end 63.946 185.936582) (width 0.2) (layer "F.Cu") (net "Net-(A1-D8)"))
 (segment (start 116.5 155.5) (end 116.5 164.6) (width 0.2) (layer "F.Cu") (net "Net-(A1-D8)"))
 (segment (start 94.546 186.554) (end 116.5 164.6) (width 0.2) (layer "F.Cu") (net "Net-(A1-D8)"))
 (segment (start 69.795635 170) (end 64.5 170) (width 0.2) (layer "F.Cu") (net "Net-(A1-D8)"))
 (segment (start 73.84 174.044365) (end 69.795635 170) (width 0.2) (layer "F.Cu") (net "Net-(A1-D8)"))
 (segment (start 77.82 174.5) (end 76.72 175.6) (width 0.2) (layer "F.Cu") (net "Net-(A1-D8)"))
 (segment (start 76.72 175.6) (end 74.824365 175.6) (width 0.2) (layer "F.Cu") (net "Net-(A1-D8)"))
 (segment (start 74.824365 175.6) (end 73.84 174.615635) (width 0.2) (layer "F.Cu") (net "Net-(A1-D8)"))
 (segment (start 64.5 170) (end 63.946 170.554) (width 0.2) (layer "F.Cu") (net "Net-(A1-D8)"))
 (segment (start 64.563418 186.554) (end 94.546 186.554) (width 0.2) (layer "F.Cu") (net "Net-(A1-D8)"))
 (segment (start 73.84 174.615635) (end 73.84 174.044365) (width 0.2) (layer "F.Cu") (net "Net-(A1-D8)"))
 (segment (start 86.164365 175.6) (end 85.52 174.955635) (width 0.2) (layer "F.Cu") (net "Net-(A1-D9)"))
 (segment (start 95.035635 175.6) (end 86.164365 175.6) (width 0.2) (layer "F.Cu") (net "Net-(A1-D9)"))
 (segment (start 121 123.4) (end 121 148.65) (width 0.2) (layer "F.Cu") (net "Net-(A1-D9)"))
 (segment (start 84.875635 173.4) (end 76.38 173.4) (width 0.2) (layer "F.Cu") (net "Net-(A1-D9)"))
 (segment (start 96.02 173.63) (end 96.02 174.615635) (width 0.2) (layer "F.Cu") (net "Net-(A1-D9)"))
 (segment (start 85.52 174.044365) (end 84.875635 173.4) (width 0.2) (layer "F.Cu") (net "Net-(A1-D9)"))
 (segment (start 76.38 173.4) (end 75.28 174.5) (width 0.2) (layer "F.Cu") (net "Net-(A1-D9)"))
 (segment (start 121 148.65) (end 96.02 173.63) (width 0.2) (layer "F.Cu") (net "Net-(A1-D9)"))
 (segment (start 85.52 174.955635) (end 85.52 174.044365) (width 0.2) (layer "F.Cu") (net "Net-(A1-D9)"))
 (segment (start 96.02 174.615635) (end 95.035635 175.6) (width 0.2) (layer "F.Cu") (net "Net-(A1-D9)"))
 (segment (start 106.525 36.395) (end 108 34.92) (width 0.2) (layer "B.Cu") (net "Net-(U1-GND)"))
 (segment (start 90.96 31.85) (end 95.505 36.395) (width 0.2) (layer "B.Cu") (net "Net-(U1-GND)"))
 (segment (start 95.505 36.395) (end 106.525 36.395) (width 0.2) (layer "B.Cu") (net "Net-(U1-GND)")))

